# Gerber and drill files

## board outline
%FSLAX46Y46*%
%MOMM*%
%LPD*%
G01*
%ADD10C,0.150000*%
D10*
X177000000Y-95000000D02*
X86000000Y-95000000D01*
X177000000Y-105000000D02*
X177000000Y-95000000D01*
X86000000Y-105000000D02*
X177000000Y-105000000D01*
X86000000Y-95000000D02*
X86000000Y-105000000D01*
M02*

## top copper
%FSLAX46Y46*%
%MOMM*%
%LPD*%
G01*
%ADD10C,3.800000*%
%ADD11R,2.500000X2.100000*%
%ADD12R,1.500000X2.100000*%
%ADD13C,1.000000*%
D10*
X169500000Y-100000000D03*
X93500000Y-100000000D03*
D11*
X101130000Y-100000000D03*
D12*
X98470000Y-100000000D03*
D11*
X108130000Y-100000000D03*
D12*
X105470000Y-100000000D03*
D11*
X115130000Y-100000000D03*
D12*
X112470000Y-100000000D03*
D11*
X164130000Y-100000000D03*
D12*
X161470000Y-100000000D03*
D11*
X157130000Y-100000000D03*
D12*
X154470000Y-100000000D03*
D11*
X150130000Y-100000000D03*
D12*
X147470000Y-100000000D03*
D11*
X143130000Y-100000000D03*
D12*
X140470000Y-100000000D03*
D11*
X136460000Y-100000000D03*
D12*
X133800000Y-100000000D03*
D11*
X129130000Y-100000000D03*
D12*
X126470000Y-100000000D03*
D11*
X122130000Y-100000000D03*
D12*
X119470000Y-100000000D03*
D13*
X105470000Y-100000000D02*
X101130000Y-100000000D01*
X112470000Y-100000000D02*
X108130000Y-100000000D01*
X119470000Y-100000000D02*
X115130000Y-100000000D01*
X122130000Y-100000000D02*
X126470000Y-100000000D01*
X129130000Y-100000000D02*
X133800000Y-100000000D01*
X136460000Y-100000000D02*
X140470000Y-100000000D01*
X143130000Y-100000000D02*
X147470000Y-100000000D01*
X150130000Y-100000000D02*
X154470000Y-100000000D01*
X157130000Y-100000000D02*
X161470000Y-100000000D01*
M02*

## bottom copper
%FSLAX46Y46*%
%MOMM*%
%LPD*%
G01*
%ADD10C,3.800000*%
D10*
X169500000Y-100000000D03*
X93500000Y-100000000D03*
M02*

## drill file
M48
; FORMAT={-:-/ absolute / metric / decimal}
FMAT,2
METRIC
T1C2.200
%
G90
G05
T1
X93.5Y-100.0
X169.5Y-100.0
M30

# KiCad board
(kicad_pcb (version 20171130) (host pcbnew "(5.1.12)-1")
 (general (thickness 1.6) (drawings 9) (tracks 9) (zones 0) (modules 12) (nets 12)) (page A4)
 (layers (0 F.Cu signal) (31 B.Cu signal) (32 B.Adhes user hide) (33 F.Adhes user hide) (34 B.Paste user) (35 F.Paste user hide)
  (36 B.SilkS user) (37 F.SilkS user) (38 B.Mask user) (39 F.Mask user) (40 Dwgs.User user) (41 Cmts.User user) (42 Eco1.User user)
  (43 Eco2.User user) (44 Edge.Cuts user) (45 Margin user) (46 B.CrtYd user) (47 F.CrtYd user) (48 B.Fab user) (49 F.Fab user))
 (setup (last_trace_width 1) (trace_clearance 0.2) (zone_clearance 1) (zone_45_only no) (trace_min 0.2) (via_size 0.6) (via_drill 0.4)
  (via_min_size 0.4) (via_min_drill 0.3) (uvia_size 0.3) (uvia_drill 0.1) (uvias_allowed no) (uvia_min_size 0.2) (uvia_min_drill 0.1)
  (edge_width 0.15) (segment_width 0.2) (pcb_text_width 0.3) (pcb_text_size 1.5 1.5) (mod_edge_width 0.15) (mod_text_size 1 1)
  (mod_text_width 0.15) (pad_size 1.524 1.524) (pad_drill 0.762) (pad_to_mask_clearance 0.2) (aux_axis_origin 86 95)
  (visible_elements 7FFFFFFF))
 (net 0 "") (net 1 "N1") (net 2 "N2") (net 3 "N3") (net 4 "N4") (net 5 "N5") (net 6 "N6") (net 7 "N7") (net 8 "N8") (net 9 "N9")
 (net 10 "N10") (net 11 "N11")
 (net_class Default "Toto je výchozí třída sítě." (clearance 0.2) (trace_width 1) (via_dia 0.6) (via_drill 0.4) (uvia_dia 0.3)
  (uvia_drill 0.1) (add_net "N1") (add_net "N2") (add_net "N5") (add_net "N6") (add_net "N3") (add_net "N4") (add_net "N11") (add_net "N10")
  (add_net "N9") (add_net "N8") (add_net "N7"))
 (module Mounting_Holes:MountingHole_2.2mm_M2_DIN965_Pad (layer F.Cu) (at 169.5 100)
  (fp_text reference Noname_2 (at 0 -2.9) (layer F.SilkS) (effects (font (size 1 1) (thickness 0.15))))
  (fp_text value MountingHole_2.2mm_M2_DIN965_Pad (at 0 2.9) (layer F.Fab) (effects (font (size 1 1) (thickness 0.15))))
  (pad 1 thru_hole circle (at 0 0) (size 3.8 3.8) (drill 2.2) (layers *.Cu *.Mask F.SilkS)))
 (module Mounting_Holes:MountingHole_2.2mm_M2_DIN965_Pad (layer F.Cu) (at 93.5 100)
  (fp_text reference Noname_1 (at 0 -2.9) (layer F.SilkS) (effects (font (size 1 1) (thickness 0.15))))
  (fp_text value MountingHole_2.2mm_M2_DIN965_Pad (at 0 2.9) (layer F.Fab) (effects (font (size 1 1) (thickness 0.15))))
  (pad 1 thru_hole circle (at 0 0) (size 3.8 3.8) (drill 2.2) (layers *.Cu *.Mask F.SilkS)))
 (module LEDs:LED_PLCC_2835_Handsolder (layer F.Cu) (at 100 100)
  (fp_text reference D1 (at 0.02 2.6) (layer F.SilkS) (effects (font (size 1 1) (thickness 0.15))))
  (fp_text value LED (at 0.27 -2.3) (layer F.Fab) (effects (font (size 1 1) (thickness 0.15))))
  (pad 1 smd rect (at 1.13 0) (size 2.5 2.1) (layers F.Cu F.Paste F.Mask) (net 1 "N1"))
  (pad 2 smd rect (at -1.53 0) (size 1.5 2.1) (layers F.Cu F.Paste F.Mask) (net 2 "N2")))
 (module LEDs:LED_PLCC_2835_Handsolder (layer F.Cu) (at 107 100)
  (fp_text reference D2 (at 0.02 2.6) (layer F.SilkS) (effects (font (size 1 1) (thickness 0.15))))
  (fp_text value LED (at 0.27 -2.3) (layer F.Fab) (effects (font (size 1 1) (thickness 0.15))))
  (pad 1 smd rect (at 1.13 0) (size 2.5 2.1) (layers F.Cu F.Paste F.Mask) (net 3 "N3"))
  (pad 2 smd rect (at -1.53 0) (size 1.5 2.1) (layers F.Cu F.Paste F.Mask) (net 1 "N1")))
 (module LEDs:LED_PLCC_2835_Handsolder (layer F.Cu) (at 114 100)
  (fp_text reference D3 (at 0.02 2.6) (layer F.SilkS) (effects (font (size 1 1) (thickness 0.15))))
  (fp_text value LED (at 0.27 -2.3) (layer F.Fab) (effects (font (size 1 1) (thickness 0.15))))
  (pad 1 smd rect (at 1.13 0) (size 2.5 2.1) (layers F.Cu F.Paste F.Mask) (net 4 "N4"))
  (pad 2 smd rect (at -1.53 0) (size 1.5 2.1) (layers F.Cu F.Paste F.Mask) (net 3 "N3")))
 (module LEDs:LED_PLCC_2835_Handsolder (layer F.Cu) (at 163 100)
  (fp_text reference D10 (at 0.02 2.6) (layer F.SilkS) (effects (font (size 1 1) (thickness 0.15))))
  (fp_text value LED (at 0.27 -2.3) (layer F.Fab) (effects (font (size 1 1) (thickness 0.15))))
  (pad 1 smd rect (at 1.13 0) (size 2.5 2.1) (layers F.Cu F.Paste F.Mask) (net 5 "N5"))
  (pad 2 smd rect (at -1.53 0) (size 1.5 2.1) (layers F.Cu F.Paste F.Mask) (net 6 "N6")))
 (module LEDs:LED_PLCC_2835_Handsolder (layer F.Cu) (at 156 100)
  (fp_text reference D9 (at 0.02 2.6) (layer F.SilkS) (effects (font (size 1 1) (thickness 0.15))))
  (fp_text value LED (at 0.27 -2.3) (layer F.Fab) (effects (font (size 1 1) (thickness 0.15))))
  (pad 1 smd rect (at 1.13 0) (size 2.5 2.1) (layers F.Cu F.Paste F.Mask) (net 6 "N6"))
  (pad 2 smd rect (at -1.53 0) (size 1.5 2.1) (layers F.Cu F.Paste F.Mask) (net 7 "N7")))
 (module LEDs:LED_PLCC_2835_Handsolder (layer F.Cu) (at 149 100)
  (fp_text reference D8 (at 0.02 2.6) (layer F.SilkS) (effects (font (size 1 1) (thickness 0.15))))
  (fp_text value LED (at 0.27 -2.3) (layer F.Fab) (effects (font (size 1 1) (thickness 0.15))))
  (pad 1 smd rect (at 1.13 0) (size 2.5 2.1) (layers F.Cu F.Paste F.Mask) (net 7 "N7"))
  (pad 2 smd rect (at -1.53 0) (size 1.5 2.1) (layers F.Cu F.Paste F.Mask) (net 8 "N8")))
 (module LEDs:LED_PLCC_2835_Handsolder (layer F.Cu) (at 142 100)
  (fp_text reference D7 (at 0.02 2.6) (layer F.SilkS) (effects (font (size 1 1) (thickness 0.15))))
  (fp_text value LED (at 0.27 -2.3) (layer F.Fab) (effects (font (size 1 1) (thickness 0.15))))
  (pad 1 smd rect (at 1.13 0) (size 2.5 2.1) (layers F.Cu F.Paste F.Mask) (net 8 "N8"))
  (pad 2 smd rect (at -1.53 0) (size 1.5 2.1) (layers F.Cu F.Paste F.Mask) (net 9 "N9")))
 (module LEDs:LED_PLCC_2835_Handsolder (layer F.Cu) (at 135.33 100)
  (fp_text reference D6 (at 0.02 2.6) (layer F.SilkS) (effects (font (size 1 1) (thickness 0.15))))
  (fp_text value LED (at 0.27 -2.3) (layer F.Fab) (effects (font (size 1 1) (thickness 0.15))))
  (pad 1 smd rect (at 1.13 0) (size 2.5 2.1) (layers F.Cu F.Paste F.Mask) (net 9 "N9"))
  (pad 2 smd rect (at -1.53 0) (size 1.5 2.1) (layers F.Cu F.Paste F.Mask) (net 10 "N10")))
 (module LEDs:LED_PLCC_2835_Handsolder (layer F.Cu) (at 128 100)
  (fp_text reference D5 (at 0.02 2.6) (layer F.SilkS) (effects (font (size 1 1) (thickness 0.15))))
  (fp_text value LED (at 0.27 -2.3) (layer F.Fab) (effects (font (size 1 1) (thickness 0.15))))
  (pad 1 smd rect (at 1.13 0) (size 2.5 2.1) (layers F.Cu F.Paste F.Mask) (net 10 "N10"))
  (pad 2 smd rect (at -1.53 0) (size 1.5 2.1) (layers F.Cu F.Paste F.Mask) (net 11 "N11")))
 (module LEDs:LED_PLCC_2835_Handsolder (layer F.Cu) (at 121 100)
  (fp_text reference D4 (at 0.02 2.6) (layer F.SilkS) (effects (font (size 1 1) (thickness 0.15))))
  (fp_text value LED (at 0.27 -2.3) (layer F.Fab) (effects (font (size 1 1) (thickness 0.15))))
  (pad 1 smd rect (at 1.13 0) (size 2.5 2.1) (layers F.Cu F.Paste F.Mask) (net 11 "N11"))
  (pad 2 smd rect (at -1.53 0) (size 1.5 2.1) (layers F.Cu F.Paste F.Mask) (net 4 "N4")))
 (gr_line (start 177 95) (end 86 95) (layer Edge.Cuts) (width 0.15))
 (gr_line (start 177 105) (end 177 95) (layer Edge.Cuts) (width 0.15))
 (gr_line (start 86 105) (end 177 105) (layer Edge.Cuts) (width 0.15))
 (gr_line (start 86 95) (end 86 105) (layer Edge.Cuts) (width 0.15))
 (segment (start 105.47 100) (end 101.13 100) (width 1) (layer F.Cu) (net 1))
 (segment (start 112.47 100) (end 108.13 100) (width 1) (layer F.Cu) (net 3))
 (segment (start 119.47 100) (end 115.13 100) (width 1) (layer F.Cu) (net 4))
 (segment (start 122.13 100) (end 126.47 100) (width 1) (layer F.Cu) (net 11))
 (segment (start 129.13 100) (end 133.8 100) (width 1) (layer F.Cu) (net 10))
 (segment (start 136.46 100) (end 140.47 100) (width 1) (layer F.Cu) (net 9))
 (segment (start 143.13 100) (end 147.47 100) (width 1) (layer F.Cu) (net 8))
 (segment (start 150.13 100) (end 154.47 100) (width 1) (layer F.Cu) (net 7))
 (segment (start 157.13 100) (end 161.47 100) (width 1) (layer F.Cu) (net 6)))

